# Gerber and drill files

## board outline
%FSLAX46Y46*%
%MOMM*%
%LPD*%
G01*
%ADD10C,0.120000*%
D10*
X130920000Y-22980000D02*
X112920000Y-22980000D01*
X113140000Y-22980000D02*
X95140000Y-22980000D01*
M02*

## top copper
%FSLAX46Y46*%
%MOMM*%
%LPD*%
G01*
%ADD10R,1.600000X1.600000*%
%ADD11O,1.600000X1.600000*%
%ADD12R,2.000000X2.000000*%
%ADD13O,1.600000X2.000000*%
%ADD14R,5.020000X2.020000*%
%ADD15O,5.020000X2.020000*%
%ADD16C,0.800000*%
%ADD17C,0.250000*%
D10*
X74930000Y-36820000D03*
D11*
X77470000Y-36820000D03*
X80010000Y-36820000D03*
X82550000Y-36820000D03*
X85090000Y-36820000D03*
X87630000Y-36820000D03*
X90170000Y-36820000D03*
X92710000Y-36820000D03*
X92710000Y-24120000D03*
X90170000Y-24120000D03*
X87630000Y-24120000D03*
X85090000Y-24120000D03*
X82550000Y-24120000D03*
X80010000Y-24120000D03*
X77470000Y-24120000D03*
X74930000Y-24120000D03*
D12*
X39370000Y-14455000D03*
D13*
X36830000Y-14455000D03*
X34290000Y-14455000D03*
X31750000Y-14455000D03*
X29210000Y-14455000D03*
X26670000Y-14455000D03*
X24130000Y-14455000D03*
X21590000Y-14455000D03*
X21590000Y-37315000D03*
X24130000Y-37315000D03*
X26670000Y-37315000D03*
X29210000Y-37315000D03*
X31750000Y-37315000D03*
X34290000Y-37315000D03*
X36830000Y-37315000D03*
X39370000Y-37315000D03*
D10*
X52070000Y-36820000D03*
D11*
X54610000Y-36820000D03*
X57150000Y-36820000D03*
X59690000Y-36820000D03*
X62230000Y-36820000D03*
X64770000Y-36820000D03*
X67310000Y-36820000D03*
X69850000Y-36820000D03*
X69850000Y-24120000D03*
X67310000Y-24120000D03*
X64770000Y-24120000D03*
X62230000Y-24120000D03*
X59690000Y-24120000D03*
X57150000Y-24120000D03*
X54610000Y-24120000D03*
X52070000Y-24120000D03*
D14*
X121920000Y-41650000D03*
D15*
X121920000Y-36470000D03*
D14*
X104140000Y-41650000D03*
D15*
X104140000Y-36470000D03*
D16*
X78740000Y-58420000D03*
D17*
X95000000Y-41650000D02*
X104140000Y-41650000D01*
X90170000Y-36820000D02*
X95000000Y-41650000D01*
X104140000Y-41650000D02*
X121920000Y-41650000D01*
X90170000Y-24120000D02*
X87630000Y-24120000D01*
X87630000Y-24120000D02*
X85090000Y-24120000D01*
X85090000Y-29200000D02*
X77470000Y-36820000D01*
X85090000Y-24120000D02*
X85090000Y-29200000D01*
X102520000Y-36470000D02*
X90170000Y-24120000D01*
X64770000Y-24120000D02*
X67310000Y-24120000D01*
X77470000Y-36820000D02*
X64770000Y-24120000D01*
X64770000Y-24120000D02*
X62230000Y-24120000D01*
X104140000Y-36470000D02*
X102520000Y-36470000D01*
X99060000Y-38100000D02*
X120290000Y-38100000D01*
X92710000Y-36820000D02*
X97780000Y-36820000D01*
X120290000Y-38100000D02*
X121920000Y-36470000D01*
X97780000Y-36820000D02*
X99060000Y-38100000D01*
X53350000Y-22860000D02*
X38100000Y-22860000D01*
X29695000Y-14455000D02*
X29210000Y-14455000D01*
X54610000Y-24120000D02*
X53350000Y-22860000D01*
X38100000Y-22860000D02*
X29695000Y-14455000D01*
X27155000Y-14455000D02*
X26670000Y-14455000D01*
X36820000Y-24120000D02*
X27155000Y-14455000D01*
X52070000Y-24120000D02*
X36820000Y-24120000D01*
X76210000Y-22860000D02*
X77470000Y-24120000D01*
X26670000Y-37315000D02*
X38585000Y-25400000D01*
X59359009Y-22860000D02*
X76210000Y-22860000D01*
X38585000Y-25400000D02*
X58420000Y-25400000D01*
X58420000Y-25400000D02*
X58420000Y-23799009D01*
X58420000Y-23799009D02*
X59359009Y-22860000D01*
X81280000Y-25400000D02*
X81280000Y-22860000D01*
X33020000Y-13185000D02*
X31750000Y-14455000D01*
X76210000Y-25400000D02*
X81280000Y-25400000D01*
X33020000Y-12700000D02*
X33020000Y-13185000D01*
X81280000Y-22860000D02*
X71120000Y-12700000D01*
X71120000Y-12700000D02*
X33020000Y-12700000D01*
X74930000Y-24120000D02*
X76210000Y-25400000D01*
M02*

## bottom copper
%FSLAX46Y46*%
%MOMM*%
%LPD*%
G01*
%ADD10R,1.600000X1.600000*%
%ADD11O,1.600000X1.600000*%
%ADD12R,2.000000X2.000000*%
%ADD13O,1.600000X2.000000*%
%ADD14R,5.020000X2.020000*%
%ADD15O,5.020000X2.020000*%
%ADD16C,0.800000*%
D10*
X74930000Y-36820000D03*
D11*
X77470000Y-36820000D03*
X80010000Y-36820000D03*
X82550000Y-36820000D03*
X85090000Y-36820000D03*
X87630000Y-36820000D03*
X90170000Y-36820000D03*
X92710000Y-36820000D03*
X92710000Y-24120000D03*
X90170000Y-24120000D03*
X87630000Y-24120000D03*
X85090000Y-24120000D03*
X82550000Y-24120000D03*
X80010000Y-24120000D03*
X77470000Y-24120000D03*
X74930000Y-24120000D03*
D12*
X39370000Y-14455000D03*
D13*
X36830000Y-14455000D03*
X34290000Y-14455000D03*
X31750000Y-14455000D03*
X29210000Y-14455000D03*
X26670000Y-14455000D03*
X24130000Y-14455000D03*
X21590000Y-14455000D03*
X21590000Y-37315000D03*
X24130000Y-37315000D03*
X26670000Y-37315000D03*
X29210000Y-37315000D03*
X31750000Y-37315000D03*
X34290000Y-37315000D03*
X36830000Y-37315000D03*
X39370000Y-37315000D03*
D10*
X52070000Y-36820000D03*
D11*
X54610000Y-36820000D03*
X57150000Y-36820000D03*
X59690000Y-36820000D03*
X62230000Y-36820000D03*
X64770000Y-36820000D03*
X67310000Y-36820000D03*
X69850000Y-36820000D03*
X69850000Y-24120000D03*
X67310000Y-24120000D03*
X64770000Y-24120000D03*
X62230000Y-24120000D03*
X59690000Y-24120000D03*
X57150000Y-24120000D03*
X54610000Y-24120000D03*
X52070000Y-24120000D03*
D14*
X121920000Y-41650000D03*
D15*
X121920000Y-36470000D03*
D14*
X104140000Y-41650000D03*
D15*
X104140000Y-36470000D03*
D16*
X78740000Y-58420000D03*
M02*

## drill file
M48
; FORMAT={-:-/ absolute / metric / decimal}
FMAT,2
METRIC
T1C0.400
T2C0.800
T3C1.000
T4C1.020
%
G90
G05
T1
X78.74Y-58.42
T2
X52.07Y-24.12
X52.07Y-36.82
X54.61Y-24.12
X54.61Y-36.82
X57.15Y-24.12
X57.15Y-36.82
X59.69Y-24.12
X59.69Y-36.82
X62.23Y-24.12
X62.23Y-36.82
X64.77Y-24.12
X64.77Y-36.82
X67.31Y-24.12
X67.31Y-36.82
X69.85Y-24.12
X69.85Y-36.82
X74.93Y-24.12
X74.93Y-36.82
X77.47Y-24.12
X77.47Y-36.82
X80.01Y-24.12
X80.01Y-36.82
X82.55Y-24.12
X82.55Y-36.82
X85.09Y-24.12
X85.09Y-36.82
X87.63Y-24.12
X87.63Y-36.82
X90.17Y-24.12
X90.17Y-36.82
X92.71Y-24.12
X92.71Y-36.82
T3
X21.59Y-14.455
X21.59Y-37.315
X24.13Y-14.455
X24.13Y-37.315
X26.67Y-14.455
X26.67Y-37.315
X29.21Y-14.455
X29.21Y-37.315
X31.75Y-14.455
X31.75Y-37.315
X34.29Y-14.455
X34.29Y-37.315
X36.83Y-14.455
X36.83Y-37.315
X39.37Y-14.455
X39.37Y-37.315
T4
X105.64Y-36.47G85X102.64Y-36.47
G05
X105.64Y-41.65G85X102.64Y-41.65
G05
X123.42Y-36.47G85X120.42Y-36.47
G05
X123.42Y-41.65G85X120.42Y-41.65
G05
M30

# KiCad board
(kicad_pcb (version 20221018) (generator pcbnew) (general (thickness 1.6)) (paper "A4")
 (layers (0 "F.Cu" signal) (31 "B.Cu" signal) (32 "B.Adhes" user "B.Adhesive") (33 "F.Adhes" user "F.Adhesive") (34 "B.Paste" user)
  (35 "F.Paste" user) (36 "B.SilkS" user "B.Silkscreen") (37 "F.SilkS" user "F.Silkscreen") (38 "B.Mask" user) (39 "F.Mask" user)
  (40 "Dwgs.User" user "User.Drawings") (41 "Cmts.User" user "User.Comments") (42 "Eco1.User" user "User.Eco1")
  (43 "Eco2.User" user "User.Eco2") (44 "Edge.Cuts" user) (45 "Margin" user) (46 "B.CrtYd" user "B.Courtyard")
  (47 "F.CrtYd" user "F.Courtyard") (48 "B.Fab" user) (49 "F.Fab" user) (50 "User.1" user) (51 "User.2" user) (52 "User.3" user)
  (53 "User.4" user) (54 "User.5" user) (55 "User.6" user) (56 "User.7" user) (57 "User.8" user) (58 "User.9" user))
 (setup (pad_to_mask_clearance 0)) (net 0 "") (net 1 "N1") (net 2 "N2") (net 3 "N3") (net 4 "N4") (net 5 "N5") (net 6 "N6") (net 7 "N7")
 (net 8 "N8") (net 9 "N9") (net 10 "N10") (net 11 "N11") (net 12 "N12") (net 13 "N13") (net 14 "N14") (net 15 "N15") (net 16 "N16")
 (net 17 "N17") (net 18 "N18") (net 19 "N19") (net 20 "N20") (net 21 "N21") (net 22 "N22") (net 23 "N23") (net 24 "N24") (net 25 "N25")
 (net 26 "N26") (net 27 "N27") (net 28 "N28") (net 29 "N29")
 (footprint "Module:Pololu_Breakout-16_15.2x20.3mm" (layer "F.Cu") (at 74.93 36.82 90)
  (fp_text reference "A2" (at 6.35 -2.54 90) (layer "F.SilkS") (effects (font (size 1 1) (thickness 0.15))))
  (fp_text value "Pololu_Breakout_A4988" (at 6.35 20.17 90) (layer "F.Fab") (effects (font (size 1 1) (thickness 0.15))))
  (pad "1" thru_hole rect (at 0 0 90) (size 1.6 1.6) (drill 0.8) (layers "*.Cu" "*.Mask") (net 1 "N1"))
  (pad "2" thru_hole oval (at 0 2.54 90) (size 1.6 1.6) (drill 0.8) (layers "*.Cu" "*.Mask") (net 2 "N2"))
  (pad "3" thru_hole oval (at 0 5.08 90) (size 1.6 1.6) (drill 0.8) (layers "*.Cu" "*.Mask") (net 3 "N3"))
  (pad "4" thru_hole oval (at 0 7.62 90) (size 1.6 1.6) (drill 0.8) (layers "*.Cu" "*.Mask") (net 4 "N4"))
  (pad "5" thru_hole oval (at 0 10.16 90) (size 1.6 1.6) (drill 0.8) (layers "*.Cu" "*.Mask") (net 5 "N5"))
  (pad "6" thru_hole oval (at 0 12.7 90) (size 1.6 1.6) (drill 0.8) (layers "*.Cu" "*.Mask") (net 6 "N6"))
  (pad "7" thru_hole oval (at 0 15.24 90) (size 1.6 1.6) (drill 0.8) (layers "*.Cu" "*.Mask") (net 1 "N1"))
  (pad "8" thru_hole oval (at 0 17.78 90) (size 1.6 1.6) (drill 0.8) (layers "*.Cu" "*.Mask") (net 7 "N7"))
  (pad "9" thru_hole oval (at 12.7 17.78 90) (size 1.6 1.6) (drill 0.8) (layers "*.Cu" "*.Mask") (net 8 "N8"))
  (pad "10" thru_hole oval (at 12.7 15.24 90) (size 1.6 1.6) (drill 0.8) (layers "*.Cu" "*.Mask") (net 2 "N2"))
  (pad "11" thru_hole oval (at 12.7 12.7 90) (size 1.6 1.6) (drill 0.8) (layers "*.Cu" "*.Mask") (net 2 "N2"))
  (pad "12" thru_hole oval (at 12.7 10.16 90) (size 1.6 1.6) (drill 0.8) (layers "*.Cu" "*.Mask") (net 2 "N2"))
  (pad "13" thru_hole oval (at 12.7 7.62 90) (size 1.6 1.6) (drill 0.8) (layers "*.Cu" "*.Mask") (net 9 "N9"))
  (pad "14" thru_hole oval (at 12.7 5.08 90) (size 1.6 1.6) (drill 0.8) (layers "*.Cu" "*.Mask") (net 9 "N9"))
  (pad "15" thru_hole oval (at 12.7 2.54 90) (size 1.6 1.6) (drill 0.8) (layers "*.Cu" "*.Mask") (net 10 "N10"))
  (pad "16" thru_hole oval (at 12.7 0 90) (size 1.6 1.6) (drill 0.8) (layers "*.Cu" "*.Mask") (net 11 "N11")))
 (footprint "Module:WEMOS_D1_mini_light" (layer "F.Cu") (at 39.37 14.455 -90)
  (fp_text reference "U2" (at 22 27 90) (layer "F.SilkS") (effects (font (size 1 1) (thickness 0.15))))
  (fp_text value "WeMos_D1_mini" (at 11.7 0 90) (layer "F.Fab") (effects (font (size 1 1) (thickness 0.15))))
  (pad "1" thru_hole rect (at 0 0 270) (size 2 2) (drill 1) (layers "*.Cu" "*.Mask") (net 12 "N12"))
  (pad "2" thru_hole oval (at 0 2.54 270) (size 2 1.6) (drill 1) (layers "*.Cu" "*.Mask") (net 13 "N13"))
  (pad "3" thru_hole oval (at 0 5.08 270) (size 2 1.6) (drill 1) (layers "*.Cu" "*.Mask") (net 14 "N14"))
  (pad "4" thru_hole oval (at 0 7.62 270) (size 2 1.6) (drill 1) (layers "*.Cu" "*.Mask") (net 11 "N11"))
  (pad "5" thru_hole oval (at 0 10.16 270) (size 2 1.6) (drill 1) (layers "*.Cu" "*.Mask") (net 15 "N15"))
  (pad "6" thru_hole oval (at 0 12.7 270) (size 2 1.6) (drill 1) (layers "*.Cu" "*.Mask") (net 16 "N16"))
  (pad "7" thru_hole oval (at 0 15.24 270) (size 2 1.6) (drill 1) (layers "*.Cu" "*.Mask") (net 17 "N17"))
  (pad "8" thru_hole oval (at 0 17.78 270) (size 2 1.6) (drill 1) (layers "*.Cu" "*.Mask") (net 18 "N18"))
  (pad "9" thru_hole oval (at 22.86 17.78 270) (size 2 1.6) (drill 1) (layers "*.Cu" "*.Mask") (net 2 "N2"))
  (pad "10" thru_hole oval (at 22.86 15.24 270) (size 2 1.6) (drill 1) (layers "*.Cu" "*.Mask") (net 1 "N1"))
  (pad "11" thru_hole oval (at 22.86 12.7 270) (size 2 1.6) (drill 1) (layers "*.Cu" "*.Mask") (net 10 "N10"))
  (pad "12" thru_hole oval (at 22.86 10.16 270) (size 2 1.6) (drill 1) (layers "*.Cu" "*.Mask") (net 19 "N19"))
  (pad "13" thru_hole oval (at 22.86 7.62 270) (size 2 1.6) (drill 1) (layers "*.Cu" "*.Mask") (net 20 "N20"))
  (pad "14" thru_hole oval (at 22.86 5.08 270) (size 2 1.6) (drill 1) (layers "*.Cu" "*.Mask") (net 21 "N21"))
  (pad "15" thru_hole oval (at 22.86 2.54 270) (size 2 1.6) (drill 1) (layers "*.Cu" "*.Mask") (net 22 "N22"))
  (pad "16" thru_hole oval (at 22.86 0 270) (size 2 1.6) (drill 1) (layers "*.Cu" "*.Mask") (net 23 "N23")))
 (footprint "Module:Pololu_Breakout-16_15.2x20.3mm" (layer "F.Cu") (at 52.07 36.82 90)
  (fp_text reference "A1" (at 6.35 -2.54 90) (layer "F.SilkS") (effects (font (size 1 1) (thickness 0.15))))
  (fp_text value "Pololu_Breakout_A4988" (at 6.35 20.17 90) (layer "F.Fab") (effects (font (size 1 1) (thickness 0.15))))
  (pad "1" thru_hole rect (at 0 0 90) (size 1.6 1.6) (drill 0.8) (layers "*.Cu" "*.Mask") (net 1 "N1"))
  (pad "2" thru_hole oval (at 0 2.54 90) (size 1.6 1.6) (drill 0.8) (layers "*.Cu" "*.Mask") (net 2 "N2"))
  (pad "3" thru_hole oval (at 0 5.08 90) (size 1.6 1.6) (drill 0.8) (layers "*.Cu" "*.Mask") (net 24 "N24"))
  (pad "4" thru_hole oval (at 0 7.62 90) (size 1.6 1.6) (drill 0.8) (layers "*.Cu" "*.Mask") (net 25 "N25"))
  (pad "5" thru_hole oval (at 0 10.16 90) (size 1.6 1.6) (drill 0.8) (layers "*.Cu" "*.Mask") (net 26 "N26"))
  (pad "6" thru_hole oval (at 0 12.7 90) (size 1.6 1.6) (drill 0.8) (layers "*.Cu" "*.Mask") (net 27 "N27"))
  (pad "7" thru_hole oval (at 0 15.24 90) (size 1.6 1.6) (drill 0.8) (layers "*.Cu" "*.Mask") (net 1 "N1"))
  (pad "8" thru_hole oval (at 0 17.78 90) (size 1.6 1.6) (drill 0.8) (layers "*.Cu" "*.Mask") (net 7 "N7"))
  (pad "9" thru_hole oval (at 12.7 17.78 90) (size 1.6 1.6) (drill 0.8) (layers "*.Cu" "*.Mask") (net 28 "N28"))
  (pad "10" thru_hole oval (at 12.7 15.24 90) (size 1.6 1.6) (drill 0.8) (layers "*.Cu" "*.Mask") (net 2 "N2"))
  (pad "11" thru_hole oval (at 12.7 12.7 90) (size 1.6 1.6) (drill 0.8) (layers "*.Cu" "*.Mask") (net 2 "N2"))
  (pad "12" thru_hole oval (at 12.7 10.16 90) (size 1.6 1.6) (drill 0.8) (layers "*.Cu" "*.Mask") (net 2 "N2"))
  (pad "13" thru_hole oval (at 12.7 7.62 90) (size 1.6 1.6) (drill 0.8) (layers "*.Cu" "*.Mask") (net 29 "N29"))
  (pad "14" thru_hole oval (at 12.7 5.08 90) (size 1.6 1.6) (drill 0.8) (layers "*.Cu" "*.Mask") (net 29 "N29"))
  (pad "15" thru_hole oval (at 12.7 2.54 90) (size 1.6 1.6) (drill 0.8) (layers "*.Cu" "*.Mask") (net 15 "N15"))
  (pad "16" thru_hole oval (at 12.7 0 90) (size 1.6 1.6) (drill 0.8) (layers "*.Cu" "*.Mask") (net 16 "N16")))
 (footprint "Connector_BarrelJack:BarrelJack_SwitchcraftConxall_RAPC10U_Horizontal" (layer "F.Cu") (at 121.92 41.65 -90)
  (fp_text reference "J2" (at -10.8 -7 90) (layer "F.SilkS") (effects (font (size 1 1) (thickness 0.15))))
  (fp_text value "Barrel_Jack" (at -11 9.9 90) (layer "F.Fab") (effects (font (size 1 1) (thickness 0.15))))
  (fp_line (start -18.67 -9) (end -18.67 9) (stroke (width 0.12) (type solid)) (layer "Edge.Cuts"))
  (pad "1" thru_hole rect (at 0 0 270) (size 2.02 5.02) (drill oval 1.02 4.02) (layers "*.Cu" "*.Mask") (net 1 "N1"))
  (pad "2" thru_hole oval (at -5.18 0 270) (size 2.02 5.02) (drill oval 1.02 4.02) (layers "*.Cu" "*.Mask") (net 7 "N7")))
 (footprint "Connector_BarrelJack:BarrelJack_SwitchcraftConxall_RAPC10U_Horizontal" (layer "F.Cu") (at 104.14 41.65 -90)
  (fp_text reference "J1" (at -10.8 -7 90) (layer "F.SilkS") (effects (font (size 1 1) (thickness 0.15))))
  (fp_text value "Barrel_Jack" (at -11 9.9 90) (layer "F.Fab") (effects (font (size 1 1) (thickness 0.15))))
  (fp_line (start -18.67 -9) (end -18.67 9) (stroke (width 0.12) (type solid)) (layer "Edge.Cuts"))
  (pad "1" thru_hole rect (at 0 0 270) (size 2.02 5.02) (drill oval 1.02 4.02) (layers "*.Cu" "*.Mask") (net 1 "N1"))
  (pad "2" thru_hole oval (at -5.18 0 270) (size 2.02 5.02) (drill oval 1.02 4.02) (layers "*.Cu" "*.Mask") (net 2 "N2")))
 (via (at 78.74 58.42) (size 0.8) (drill 0.4) (layers "F.Cu" "B.Cu") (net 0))
 (segment (start 95 41.65) (end 104.14 41.65) (width 0.25) (layer "F.Cu") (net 1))
 (segment (start 90.17 36.82) (end 95 41.65) (width 0.25) (layer "F.Cu") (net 1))
 (segment (start 104.14 41.65) (end 121.92 41.65) (width 0.25) (layer "F.Cu") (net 1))
 (segment (start 90.17 24.12) (end 87.63 24.12) (width 0.25) (layer "F.Cu") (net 2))
 (segment (start 87.63 24.12) (end 85.09 24.12) (width 0.25) (layer "F.Cu") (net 2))
 (segment (start 85.09 29.2) (end 77.47 36.82) (width 0.25) (layer "F.Cu") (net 2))
 (segment (start 85.09 24.12) (end 85.09 29.2) (width 0.25) (layer "F.Cu") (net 2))
 (segment (start 102.52 36.47) (end 90.17 24.12) (width 0.25) (layer "F.Cu") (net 2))
 (segment (start 64.77 24.12) (end 67.31 24.12) (width 0.25) (layer "F.Cu") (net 2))
 (segment (start 77.47 36.82) (end 64.77 24.12) (width 0.25) (layer "F.Cu") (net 2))
 (segment (start 64.77 24.12) (end 62.23 24.12) (width 0.25) (layer "F.Cu") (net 2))
 (segment (start 104.14 36.47) (end 102.52 36.47) (width 0.25) (layer "F.Cu") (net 2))
 (segment (start 99.06 38.1) (end 120.29 38.1) (width 0.25) (layer "F.Cu") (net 7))
 (segment (start 92.71 36.82) (end 97.78 36.82) (width 0.25) (layer "F.Cu") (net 7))
 (segment (start 120.29 38.1) (end 121.92 36.47) (width 0.25) (layer "F.Cu") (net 7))
 (segment (start 97.78 36.82) (end 99.06 38.1) (width 0.25) (layer "F.Cu") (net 7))
 (segment (start 53.35 22.86) (end 38.1 22.86) (width 0.25) (layer "F.Cu") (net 15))
 (segment (start 29.695 14.455) (end 29.21 14.455) (width 0.25) (layer "F.Cu") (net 15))
 (segment (start 54.61 24.12) (end 53.35 22.86) (width 0.25) (layer "F.Cu") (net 15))
 (segment (start 38.1 22.86) (end 29.695 14.455) (width 0.25) (layer "F.Cu") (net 15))
 (segment (start 27.155 14.455) (end 26.67 14.455) (width 0.25) (layer "F.Cu") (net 16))
 (segment (start 36.82 24.12) (end 27.155 14.455) (width 0.25) (layer "F.Cu") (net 16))
 (segment (start 52.07 24.12) (end 36.82 24.12) (width 0.25) (layer "F.Cu") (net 16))
 (segment (start 76.21 22.86) (end 77.47 24.12) (width 0.25) (layer "F.Cu") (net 10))
 (segment (start 26.67 37.315) (end 38.585 25.4) (width 0.25) (layer "F.Cu") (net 10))
 (segment (start 59.359009 22.86) (end 76.21 22.86) (width 0.25) (layer "F.Cu") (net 10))
 (segment (start 38.585 25.4) (end 58.42 25.4) (width 0.25) (layer "F.Cu") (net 10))
 (segment (start 58.42 25.4) (end 58.42 23.799009) (width 0.25) (layer "F.Cu") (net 10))
 (segment (start 58.42 23.799009) (end 59.359009 22.86) (width 0.25) (layer "F.Cu") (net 10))
 (segment (start 81.28 25.4) (end 81.28 22.86) (width 0.25) (layer "F.Cu") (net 11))
 (segment (start 33.02 13.185) (end 31.75 14.455) (width 0.25) (layer "F.Cu") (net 11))
 (segment (start 76.21 25.4) (end 81.28 25.4) (width 0.25) (layer "F.Cu") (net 11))
 (segment (start 33.02 12.7) (end 33.02 13.185) (width 0.25) (layer "F.Cu") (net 11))
 (segment (start 81.28 22.86) (end 71.12 12.7) (width 0.25) (layer "F.Cu") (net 11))
 (segment (start 71.12 12.7) (end 33.02 12.7) (width 0.25) (layer "F.Cu") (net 11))
 (segment (start 74.93 24.12) (end 76.21 25.4) (width 0.25) (layer "F.Cu") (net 11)))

